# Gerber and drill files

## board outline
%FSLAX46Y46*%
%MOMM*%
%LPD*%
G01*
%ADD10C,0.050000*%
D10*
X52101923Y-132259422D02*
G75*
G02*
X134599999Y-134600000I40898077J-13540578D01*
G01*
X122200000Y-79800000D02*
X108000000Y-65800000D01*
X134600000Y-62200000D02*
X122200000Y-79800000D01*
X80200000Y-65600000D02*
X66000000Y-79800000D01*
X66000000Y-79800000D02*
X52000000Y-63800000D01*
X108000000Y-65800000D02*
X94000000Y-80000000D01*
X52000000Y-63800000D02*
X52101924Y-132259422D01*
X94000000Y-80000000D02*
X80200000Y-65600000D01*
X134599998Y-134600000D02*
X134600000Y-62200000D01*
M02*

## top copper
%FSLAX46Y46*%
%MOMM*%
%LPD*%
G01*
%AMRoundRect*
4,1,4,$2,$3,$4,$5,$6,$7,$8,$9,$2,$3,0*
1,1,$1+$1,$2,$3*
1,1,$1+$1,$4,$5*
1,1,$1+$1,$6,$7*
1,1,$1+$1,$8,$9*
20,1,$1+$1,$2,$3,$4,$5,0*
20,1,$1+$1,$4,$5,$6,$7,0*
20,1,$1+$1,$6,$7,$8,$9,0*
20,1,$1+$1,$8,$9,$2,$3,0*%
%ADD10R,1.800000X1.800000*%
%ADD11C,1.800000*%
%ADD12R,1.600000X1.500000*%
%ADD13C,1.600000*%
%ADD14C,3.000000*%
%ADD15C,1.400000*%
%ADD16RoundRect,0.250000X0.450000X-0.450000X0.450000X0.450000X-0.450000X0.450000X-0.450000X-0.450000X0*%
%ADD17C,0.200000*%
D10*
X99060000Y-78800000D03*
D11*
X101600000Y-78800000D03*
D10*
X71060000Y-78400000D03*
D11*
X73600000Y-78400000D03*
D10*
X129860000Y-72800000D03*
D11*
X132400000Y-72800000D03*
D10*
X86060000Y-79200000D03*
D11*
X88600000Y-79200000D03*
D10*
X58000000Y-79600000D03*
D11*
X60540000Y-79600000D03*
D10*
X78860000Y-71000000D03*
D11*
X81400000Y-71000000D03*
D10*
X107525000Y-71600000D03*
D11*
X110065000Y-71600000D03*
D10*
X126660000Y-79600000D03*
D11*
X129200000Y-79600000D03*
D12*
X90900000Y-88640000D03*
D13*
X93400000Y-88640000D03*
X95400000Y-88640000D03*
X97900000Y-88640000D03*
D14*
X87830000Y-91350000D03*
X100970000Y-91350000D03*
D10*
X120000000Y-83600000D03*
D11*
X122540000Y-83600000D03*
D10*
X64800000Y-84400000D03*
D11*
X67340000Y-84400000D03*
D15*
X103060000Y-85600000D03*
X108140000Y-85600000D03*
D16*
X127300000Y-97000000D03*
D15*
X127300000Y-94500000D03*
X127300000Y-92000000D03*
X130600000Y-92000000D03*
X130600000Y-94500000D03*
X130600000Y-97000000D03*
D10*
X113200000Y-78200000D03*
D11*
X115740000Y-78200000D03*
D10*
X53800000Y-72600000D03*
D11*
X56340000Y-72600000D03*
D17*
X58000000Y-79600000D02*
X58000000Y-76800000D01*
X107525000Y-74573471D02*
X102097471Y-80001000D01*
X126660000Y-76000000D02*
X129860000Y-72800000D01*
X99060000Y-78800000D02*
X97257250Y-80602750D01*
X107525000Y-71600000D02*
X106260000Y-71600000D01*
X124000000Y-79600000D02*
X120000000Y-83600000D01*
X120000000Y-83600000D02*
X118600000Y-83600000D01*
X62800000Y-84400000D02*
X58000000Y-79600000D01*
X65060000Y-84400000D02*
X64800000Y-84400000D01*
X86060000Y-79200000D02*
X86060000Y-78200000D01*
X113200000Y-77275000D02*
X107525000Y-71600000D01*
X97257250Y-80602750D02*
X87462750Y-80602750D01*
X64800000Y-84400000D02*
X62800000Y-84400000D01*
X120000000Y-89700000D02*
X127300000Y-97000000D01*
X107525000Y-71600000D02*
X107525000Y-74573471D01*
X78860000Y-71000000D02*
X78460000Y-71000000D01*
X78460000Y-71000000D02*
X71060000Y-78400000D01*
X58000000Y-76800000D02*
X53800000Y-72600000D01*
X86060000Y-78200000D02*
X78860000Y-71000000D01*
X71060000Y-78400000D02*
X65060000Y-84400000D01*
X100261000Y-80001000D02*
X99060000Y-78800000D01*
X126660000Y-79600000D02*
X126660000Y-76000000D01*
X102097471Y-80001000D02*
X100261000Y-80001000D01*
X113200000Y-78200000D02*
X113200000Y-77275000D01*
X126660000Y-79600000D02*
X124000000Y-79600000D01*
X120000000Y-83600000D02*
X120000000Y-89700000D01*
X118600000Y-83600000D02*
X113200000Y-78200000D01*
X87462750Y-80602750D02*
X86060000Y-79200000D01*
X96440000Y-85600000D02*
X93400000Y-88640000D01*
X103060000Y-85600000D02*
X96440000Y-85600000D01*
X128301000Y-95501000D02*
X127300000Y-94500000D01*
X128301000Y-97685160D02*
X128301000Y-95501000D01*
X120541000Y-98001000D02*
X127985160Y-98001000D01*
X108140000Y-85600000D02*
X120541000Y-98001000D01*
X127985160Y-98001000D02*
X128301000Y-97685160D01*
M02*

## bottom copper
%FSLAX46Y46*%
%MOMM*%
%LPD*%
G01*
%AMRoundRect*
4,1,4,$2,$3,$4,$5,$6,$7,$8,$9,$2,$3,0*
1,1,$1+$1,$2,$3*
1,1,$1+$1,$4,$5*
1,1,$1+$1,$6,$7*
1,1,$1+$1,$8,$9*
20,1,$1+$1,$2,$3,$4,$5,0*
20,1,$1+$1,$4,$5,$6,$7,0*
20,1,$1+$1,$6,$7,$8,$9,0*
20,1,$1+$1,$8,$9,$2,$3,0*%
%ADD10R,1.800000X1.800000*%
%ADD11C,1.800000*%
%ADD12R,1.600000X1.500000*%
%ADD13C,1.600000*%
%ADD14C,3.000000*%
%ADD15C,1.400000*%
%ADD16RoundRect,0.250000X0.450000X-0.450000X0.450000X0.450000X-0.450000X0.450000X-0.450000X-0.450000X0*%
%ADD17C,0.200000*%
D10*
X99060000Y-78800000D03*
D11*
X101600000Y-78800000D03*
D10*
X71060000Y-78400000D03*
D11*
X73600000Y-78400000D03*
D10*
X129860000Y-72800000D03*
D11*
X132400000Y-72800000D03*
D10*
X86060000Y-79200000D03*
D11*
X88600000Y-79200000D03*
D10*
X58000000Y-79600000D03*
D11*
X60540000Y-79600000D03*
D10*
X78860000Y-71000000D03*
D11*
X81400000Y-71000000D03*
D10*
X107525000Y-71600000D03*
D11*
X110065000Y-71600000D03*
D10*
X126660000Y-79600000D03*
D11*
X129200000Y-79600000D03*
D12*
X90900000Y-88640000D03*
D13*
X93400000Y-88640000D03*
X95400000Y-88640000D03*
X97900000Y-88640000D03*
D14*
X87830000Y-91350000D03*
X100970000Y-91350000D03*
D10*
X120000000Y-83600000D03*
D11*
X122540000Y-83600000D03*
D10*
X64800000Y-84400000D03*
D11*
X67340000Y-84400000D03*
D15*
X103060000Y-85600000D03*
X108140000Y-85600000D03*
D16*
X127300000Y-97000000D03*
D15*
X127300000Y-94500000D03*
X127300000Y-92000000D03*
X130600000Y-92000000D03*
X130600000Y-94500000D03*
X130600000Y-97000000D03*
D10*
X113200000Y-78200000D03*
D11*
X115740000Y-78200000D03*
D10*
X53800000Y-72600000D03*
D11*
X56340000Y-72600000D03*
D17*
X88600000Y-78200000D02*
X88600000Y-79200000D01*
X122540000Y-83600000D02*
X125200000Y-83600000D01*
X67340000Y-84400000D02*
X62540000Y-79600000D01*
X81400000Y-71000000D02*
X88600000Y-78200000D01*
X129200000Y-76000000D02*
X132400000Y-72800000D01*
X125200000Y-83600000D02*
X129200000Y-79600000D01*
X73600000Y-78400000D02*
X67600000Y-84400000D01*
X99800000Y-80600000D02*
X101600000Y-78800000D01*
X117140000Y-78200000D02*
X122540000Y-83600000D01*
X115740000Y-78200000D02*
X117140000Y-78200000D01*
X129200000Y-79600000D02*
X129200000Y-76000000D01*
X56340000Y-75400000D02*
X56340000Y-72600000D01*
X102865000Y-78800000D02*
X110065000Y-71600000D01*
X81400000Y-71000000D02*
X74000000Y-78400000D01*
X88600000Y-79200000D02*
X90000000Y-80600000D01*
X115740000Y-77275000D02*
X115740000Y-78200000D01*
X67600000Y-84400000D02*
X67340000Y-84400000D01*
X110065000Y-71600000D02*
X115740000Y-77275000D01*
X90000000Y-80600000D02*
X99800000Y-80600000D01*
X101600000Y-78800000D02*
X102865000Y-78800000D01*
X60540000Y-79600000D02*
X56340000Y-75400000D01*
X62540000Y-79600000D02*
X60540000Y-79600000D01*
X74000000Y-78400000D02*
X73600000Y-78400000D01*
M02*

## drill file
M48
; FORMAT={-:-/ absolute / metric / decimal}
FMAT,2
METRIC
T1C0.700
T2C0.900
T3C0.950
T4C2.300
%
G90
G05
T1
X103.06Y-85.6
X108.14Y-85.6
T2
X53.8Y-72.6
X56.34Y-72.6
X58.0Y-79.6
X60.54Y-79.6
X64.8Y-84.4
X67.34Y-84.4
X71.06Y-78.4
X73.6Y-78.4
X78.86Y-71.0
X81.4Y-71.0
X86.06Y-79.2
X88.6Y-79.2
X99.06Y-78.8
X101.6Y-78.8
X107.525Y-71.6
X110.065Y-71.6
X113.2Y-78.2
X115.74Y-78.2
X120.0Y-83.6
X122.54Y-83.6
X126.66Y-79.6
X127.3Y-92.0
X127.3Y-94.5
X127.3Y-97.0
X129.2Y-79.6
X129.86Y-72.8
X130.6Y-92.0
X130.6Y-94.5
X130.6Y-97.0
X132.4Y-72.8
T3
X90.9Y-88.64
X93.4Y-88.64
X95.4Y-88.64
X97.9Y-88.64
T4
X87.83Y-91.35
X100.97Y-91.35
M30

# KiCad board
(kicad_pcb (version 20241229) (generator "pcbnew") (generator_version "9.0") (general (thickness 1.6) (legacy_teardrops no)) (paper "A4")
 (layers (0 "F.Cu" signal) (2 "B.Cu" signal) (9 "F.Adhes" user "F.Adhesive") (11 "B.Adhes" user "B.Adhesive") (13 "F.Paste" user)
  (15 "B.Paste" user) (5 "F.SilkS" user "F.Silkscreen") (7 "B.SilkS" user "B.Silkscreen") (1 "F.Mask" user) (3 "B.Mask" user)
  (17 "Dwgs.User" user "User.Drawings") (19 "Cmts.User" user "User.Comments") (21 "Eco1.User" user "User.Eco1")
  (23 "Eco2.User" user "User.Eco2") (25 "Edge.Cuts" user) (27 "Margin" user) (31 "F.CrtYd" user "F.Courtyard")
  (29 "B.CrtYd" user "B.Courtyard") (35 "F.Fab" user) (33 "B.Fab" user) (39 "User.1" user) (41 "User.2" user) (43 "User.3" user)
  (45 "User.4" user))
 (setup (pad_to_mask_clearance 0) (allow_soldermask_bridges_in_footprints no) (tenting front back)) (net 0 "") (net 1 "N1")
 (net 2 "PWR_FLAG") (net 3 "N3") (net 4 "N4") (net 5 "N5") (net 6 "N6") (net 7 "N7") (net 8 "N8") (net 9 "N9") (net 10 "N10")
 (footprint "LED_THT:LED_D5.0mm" (layer "F.Cu") (at 99.06 78.8)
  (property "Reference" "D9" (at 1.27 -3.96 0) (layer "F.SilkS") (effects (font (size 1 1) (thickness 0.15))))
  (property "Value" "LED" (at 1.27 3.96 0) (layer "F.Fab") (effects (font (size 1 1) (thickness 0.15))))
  (pad "1" thru_hole rect (at 0 0) (size 1.8 1.8) (drill 0.9) (layers "*.Cu" "*.Mask") (remove_unused_layers no) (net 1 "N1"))
  (pad "2" thru_hole circle (at 2.54 0) (size 1.8 1.8) (drill 0.9) (layers "*.Cu" "*.Mask") (remove_unused_layers no) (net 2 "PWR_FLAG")))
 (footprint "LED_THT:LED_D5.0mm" (layer "F.Cu") (at 71.06 78.4)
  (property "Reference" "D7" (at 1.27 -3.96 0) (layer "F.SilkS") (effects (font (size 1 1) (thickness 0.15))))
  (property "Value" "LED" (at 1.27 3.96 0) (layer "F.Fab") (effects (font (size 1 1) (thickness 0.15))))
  (pad "1" thru_hole rect (at 0 0) (size 1.8 1.8) (drill 0.9) (layers "*.Cu" "*.Mask") (remove_unused_layers no) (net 1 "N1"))
  (pad "2" thru_hole circle (at 2.54 0) (size 1.8 1.8) (drill 0.9) (layers "*.Cu" "*.Mask") (remove_unused_layers no) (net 2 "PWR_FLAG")))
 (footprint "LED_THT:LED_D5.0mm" (layer "F.Cu") (at 129.86 72.8)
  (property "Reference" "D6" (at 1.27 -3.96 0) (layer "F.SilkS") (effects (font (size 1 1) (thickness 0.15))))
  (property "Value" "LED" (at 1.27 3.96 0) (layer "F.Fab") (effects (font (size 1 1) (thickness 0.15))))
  (pad "1" thru_hole rect (at 0 0) (size 1.8 1.8) (drill 0.9) (layers "*.Cu" "*.Mask") (remove_unused_layers no) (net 1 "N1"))
  (pad "2" thru_hole circle (at 2.54 0) (size 1.8 1.8) (drill 0.9) (layers "*.Cu" "*.Mask") (remove_unused_layers no) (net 2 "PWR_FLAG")))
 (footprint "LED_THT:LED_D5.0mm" (layer "F.Cu") (at 86.06 79.2)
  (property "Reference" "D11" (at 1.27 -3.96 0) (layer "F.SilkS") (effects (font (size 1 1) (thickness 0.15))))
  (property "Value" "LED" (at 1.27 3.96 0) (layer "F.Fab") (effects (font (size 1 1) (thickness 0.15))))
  (pad "1" thru_hole rect (at 0 0) (size 1.8 1.8) (drill 0.9) (layers "*.Cu" "*.Mask") (remove_unused_layers no) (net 1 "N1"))
  (pad "2" thru_hole circle (at 2.54 0) (size 1.8 1.8) (drill 0.9) (layers "*.Cu" "*.Mask") (remove_unused_layers no) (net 2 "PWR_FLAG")))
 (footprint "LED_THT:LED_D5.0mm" (layer "F.Cu") (at 58 79.6)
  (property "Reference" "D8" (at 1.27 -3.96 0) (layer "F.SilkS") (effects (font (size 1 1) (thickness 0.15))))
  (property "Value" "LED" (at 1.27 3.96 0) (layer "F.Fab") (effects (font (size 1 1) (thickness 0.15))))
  (pad "1" thru_hole rect (at 0 0) (size 1.8 1.8) (drill 0.9) (layers "*.Cu" "*.Mask") (remove_unused_layers no) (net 1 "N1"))
  (pad "2" thru_hole circle (at 2.54 0) (size 1.8 1.8) (drill 0.9) (layers "*.Cu" "*.Mask") (remove_unused_layers no) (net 2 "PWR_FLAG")))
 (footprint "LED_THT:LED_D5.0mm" (layer "F.Cu") (at 78.86 71)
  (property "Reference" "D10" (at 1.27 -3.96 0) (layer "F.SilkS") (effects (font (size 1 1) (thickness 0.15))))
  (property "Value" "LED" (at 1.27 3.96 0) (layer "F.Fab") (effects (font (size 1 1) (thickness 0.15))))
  (pad "1" thru_hole rect (at 0 0) (size 1.8 1.8) (drill 0.9) (layers "*.Cu" "*.Mask") (remove_unused_layers no) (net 1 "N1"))
  (pad "2" thru_hole circle (at 2.54 0) (size 1.8 1.8) (drill 0.9) (layers "*.Cu" "*.Mask") (remove_unused_layers no) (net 2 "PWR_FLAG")))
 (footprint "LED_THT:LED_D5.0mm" (layer "F.Cu") (at 107.525 71.6)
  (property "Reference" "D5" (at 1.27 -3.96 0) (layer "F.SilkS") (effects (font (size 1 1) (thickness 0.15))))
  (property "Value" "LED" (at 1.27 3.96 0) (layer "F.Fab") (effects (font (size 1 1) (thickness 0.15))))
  (pad "1" thru_hole rect (at 0 0) (size 1.8 1.8) (drill 0.9) (layers "*.Cu" "*.Mask") (remove_unused_layers no) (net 1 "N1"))
  (pad "2" thru_hole circle (at 2.54 0) (size 1.8 1.8) (drill 0.9) (layers "*.Cu" "*.Mask") (remove_unused_layers no) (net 2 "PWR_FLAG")))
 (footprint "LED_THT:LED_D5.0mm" (layer "F.Cu") (at 126.66 79.6)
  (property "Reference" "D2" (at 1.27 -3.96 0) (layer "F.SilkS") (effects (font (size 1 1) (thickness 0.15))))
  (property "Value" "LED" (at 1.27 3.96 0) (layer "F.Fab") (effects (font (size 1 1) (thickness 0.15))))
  (pad "1" thru_hole rect (at 0 0) (size 1.8 1.8) (drill 0.9) (layers "*.Cu" "*.Mask") (remove_unused_layers no) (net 1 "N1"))
  (pad "2" thru_hole circle (at 2.54 0) (size 1.8 1.8) (drill 0.9) (layers "*.Cu" "*.Mask") (remove_unused_layers no) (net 2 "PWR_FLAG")))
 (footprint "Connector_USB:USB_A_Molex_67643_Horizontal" (layer "F.Cu") (at 90.9 88.64)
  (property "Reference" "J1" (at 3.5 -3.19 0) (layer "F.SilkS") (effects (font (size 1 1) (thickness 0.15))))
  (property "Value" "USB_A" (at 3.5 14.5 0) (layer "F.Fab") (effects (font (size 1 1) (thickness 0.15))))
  (pad "1" thru_hole rect (at 0 0) (size 1.6 1.5) (drill 0.95) (layers "*.Cu" "*.Mask") (remove_unused_layers no) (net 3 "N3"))
  (pad "2" thru_hole circle (at 2.5 0) (size 1.6 1.6) (drill 0.95) (layers "*.Cu" "*.Mask") (remove_unused_layers no) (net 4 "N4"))
  (pad "3" thru_hole circle (at 4.5 0) (size 1.6 1.6) (drill 0.95) (layers "*.Cu" "*.Mask") (remove_unused_layers no) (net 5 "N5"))
  (pad "4" thru_hole circle (at 7 0) (size 1.6 1.6) (drill 0.95) (layers "*.Cu" "*.Mask") (remove_unused_layers no) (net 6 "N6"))
  (pad "5" thru_hole circle (at -3.07 2.71) (size 3 3) (drill 2.3) (layers "*.Cu" "*.Mask") (remove_unused_layers no) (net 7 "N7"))
  (pad "5" thru_hole circle (at 10.07 2.71) (size 3 3) (drill 2.3) (layers "*.Cu" "*.Mask") (remove_unused_layers no) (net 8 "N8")))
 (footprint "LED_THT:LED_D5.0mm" (layer "F.Cu") (at 120 83.6)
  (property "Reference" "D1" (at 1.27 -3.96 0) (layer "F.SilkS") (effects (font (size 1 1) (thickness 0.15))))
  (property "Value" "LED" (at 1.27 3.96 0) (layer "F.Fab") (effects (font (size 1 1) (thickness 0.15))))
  (pad "1" thru_hole rect (at 0 0) (size 1.8 1.8) (drill 0.9) (layers "*.Cu" "*.Mask") (remove_unused_layers no) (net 1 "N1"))
  (pad "2" thru_hole circle (at 2.54 0) (size 1.8 1.8) (drill 0.9) (layers "*.Cu" "*.Mask") (remove_unused_layers no) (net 2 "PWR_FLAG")))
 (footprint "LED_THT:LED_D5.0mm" (layer "F.Cu") (at 64.8 84.4)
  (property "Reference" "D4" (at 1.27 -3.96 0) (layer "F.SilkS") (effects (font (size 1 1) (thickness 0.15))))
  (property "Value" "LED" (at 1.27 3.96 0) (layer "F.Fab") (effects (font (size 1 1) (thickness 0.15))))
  (pad "1" thru_hole rect (at 0 0) (size 1.8 1.8) (drill 0.9) (layers "*.Cu" "*.Mask") (remove_unused_layers no) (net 1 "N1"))
  (pad "2" thru_hole circle (at 2.54 0) (size 1.8 1.8) (drill 0.9) (layers "*.Cu" "*.Mask") (remove_unused_layers no) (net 2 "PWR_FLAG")))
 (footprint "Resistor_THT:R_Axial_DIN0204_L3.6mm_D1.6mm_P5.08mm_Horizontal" (layer "F.Cu") (at 103.06 85.6)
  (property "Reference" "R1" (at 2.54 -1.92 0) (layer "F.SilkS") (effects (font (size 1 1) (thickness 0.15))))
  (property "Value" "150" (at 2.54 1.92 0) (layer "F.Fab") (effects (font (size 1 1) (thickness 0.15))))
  (pad "1" thru_hole circle (at 0 0) (size 1.4 1.4) (drill 0.7) (layers "*.Cu" "*.Mask") (remove_unused_layers no) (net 4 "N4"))
  (pad "2" thru_hole circle (at 5.08 0) (size 1.4 1.4) (drill 0.7) (layers "*.Cu" "*.Mask") (remove_unused_layers no) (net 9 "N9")))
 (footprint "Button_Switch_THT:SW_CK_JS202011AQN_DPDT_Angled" (layer "F.Cu") (at 127.3 97 90)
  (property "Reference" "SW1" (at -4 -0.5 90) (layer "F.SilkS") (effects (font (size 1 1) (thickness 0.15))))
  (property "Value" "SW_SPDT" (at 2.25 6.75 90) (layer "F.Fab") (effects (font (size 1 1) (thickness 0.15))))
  (pad "1" thru_hole roundrect (at 0 0 90) (size 1.4 1.4) (drill 0.9) (layers "*.Cu" "*.Mask") (remove_unused_layers no)
   (roundrect_rratio 0.1785714286) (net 1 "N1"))
  (pad "2" thru_hole circle (at 2.5 0 90) (size 1.4 1.4) (drill 0.9) (layers "*.Cu" "*.Mask") (remove_unused_layers no) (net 9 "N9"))
  (pad "3" thru_hole circle (at 5 0 90) (size 1.4 1.4) (drill 0.9) (layers "*.Cu" "*.Mask") (remove_unused_layers no) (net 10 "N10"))
  (pad "4" thru_hole circle (at 5 3.3 90) (size 1.4 1.4) (drill 0.9) (layers "*.Cu" "*.Mask") (remove_unused_layers no))
  (pad "5" thru_hole circle (at 2.5 3.3 90) (size 1.4 1.4) (drill 0.9) (layers "*.Cu" "*.Mask") (remove_unused_layers no))
  (pad "6" thru_hole circle (at 0 3.3 90) (size 1.4 1.4) (drill 0.9) (layers "*.Cu" "*.Mask") (remove_unused_layers no)))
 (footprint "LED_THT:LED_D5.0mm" (layer "F.Cu") (at 113.2 78.2)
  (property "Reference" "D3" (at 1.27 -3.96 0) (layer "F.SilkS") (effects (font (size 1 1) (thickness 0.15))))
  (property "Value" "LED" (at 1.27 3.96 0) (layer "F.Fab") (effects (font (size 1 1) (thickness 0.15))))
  (pad "1" thru_hole rect (at 0 0) (size 1.8 1.8) (drill 0.9) (layers "*.Cu" "*.Mask") (remove_unused_layers no) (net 1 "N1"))
  (pad "2" thru_hole circle (at 2.54 0) (size 1.8 1.8) (drill 0.9) (layers "*.Cu" "*.Mask") (remove_unused_layers no) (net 2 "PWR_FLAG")))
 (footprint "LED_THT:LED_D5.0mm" (layer "F.Cu") (at 53.8 72.6)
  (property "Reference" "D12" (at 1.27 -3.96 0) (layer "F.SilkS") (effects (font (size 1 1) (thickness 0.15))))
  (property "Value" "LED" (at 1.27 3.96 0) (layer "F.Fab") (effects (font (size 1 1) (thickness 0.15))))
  (pad "1" thru_hole rect (at 0 0) (size 1.8 1.8) (drill 0.9) (layers "*.Cu" "*.Mask") (remove_unused_layers no) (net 1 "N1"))
  (pad "2" thru_hole circle (at 2.54 0) (size 1.8 1.8) (drill 0.9) (layers "*.Cu" "*.Mask") (remove_unused_layers no) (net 2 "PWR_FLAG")))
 (gr_arc (start 52.101923 132.259422) (mid 94.221782 102.73601) (end 134.6 134.6) (stroke (width 0.05) (type default)) (layer "Edge.Cuts"))
 (gr_line (start 122.2 79.8) (end 108 65.8) (stroke (width 0.05) (type default)) (layer "Edge.Cuts"))
 (gr_line (start 134.6 62.2) (end 122.2 79.8) (stroke (width 0.05) (type default)) (layer "Edge.Cuts"))
 (gr_line (start 80.2 65.6) (end 66 79.8) (stroke (width 0.05) (type default)) (layer "Edge.Cuts"))
 (gr_line (start 66 79.8) (end 52 63.8) (stroke (width 0.05) (type default)) (layer "Edge.Cuts"))
 (gr_line (start 108 65.8) (end 94 80) (stroke (width 0.05) (type default)) (layer "Edge.Cuts"))
 (gr_line (start 52 63.8) (end 52.101924 132.259422) (stroke (width 0.05) (type default)) (layer "Edge.Cuts"))
 (gr_line (start 94 80) (end 80.2 65.6) (stroke (width 0.05) (type default)) (layer "Edge.Cuts"))
 (gr_line (start 134.599998 134.6) (end 134.6 62.2) (stroke (width 0.05) (type default)) (layer "Edge.Cuts"))
 (segment (start 88.6 78.2) (end 88.6 79.2) (width 0.2) (layer "B.Cu") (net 2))
 (segment (start 122.54 83.6) (end 125.2 83.6) (width 0.2) (layer "B.Cu") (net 2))
 (segment (start 67.34 84.4) (end 62.54 79.6) (width 0.2) (layer "B.Cu") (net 2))
 (segment (start 81.4 71) (end 88.6 78.2) (width 0.2) (layer "B.Cu") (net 2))
 (segment (start 129.2 76) (end 132.4 72.8) (width 0.2) (layer "B.Cu") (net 2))
 (segment (start 125.2 83.6) (end 129.2 79.6) (width 0.2) (layer "B.Cu") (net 2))
 (segment (start 73.6 78.4) (end 67.6 84.4) (width 0.2) (layer "B.Cu") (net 2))
 (segment (start 99.8 80.6) (end 101.6 78.8) (width 0.2) (layer "B.Cu") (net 2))
 (segment (start 117.14 78.2) (end 122.54 83.6) (width 0.2) (layer "B.Cu") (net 2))
 (segment (start 115.74 78.2) (end 117.14 78.2) (width 0.2) (layer "B.Cu") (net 2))
 (segment (start 129.2 79.6) (end 129.2 76) (width 0.2) (layer "B.Cu") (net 2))
 (segment (start 56.34 75.4) (end 56.34 72.6) (width 0.2) (layer "B.Cu") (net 2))
 (segment (start 102.865 78.8) (end 110.065 71.6) (width 0.2) (layer "B.Cu") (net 2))
 (segment (start 81.4 71) (end 74 78.4) (width 0.2) (layer "B.Cu") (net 2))
 (segment (start 88.6 79.2) (end 90 80.6) (width 0.2) (layer "B.Cu") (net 2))
 (segment (start 115.74 77.275) (end 115.74 78.2) (width 0.2) (layer "B.Cu") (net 2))
 (segment (start 67.6 84.4) (end 67.34 84.4) (width 0.2) (layer "B.Cu") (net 2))
 (segment (start 110.065 71.6) (end 115.74 77.275) (width 0.2) (layer "B.Cu") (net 2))
 (segment (start 90 80.6) (end 99.8 80.6) (width 0.2) (layer "B.Cu") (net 2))
 (segment (start 101.6 78.8) (end 102.865 78.8) (width 0.2) (layer "B.Cu") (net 2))
 (segment (start 60.54 79.6) (end 56.34 75.4) (width 0.2) (layer "B.Cu") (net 2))
 (segment (start 62.54 79.6) (end 60.54 79.6) (width 0.2) (layer "B.Cu") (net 2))
 (segment (start 74 78.4) (end 73.6 78.4) (width 0.2) (layer "B.Cu") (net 2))
 (segment (start 58 79.6) (end 58 76.8) (width 0.2) (layer "F.Cu") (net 1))
 (segment (start 107.525 74.573471) (end 102.097471 80.001) (width 0.2) (layer "F.Cu") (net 1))
 (segment (start 126.66 76) (end 129.86 72.8) (width 0.2) (layer "F.Cu") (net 1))
 (segment (start 99.06 78.8) (end 97.25725 80.60275) (width 0.2) (layer "F.Cu") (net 1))
 (segment (start 107.525 71.6) (end 106.26 71.6) (width 0.2) (layer "F.Cu") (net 1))
 (segment (start 124 79.6) (end 120 83.6) (width 0.2) (layer "F.Cu") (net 1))
 (segment (start 120 83.6) (end 118.6 83.6) (width 0.2) (layer "F.Cu") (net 1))
 (segment (start 62.8 84.4) (end 58 79.6) (width 0.2) (layer "F.Cu") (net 1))
 (segment (start 65.06 84.4) (end 64.8 84.4) (width 0.2) (layer "F.Cu") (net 1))
 (segment (start 86.06 79.2) (end 86.06 78.2) (width 0.2) (layer "F.Cu") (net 1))
 (segment (start 113.2 77.275) (end 107.525 71.6) (width 0.2) (layer "F.Cu") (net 1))
 (segment (start 97.25725 80.60275) (end 87.46275 80.60275) (width 0.2) (layer "F.Cu") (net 1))
 (segment (start 64.8 84.4) (end 62.8 84.4) (width 0.2) (layer "F.Cu") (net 1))
 (segment (start 120 89.7) (end 127.3 97) (width 0.2) (layer "F.Cu") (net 1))
 (segment (start 107.525 71.6) (end 107.525 74.573471) (width 0.2) (layer "F.Cu") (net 1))
 (segment (start 78.86 71) (end 78.46 71) (width 0.2) (layer "F.Cu") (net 1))
 (segment (start 78.46 71) (end 71.06 78.4) (width 0.2) (layer "F.Cu") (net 1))
 (segment (start 58 76.8) (end 53.8 72.6) (width 0.2) (layer "F.Cu") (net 1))
 (segment (start 86.06 78.2) (end 78.86 71) (width 0.2) (layer "F.Cu") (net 1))
 (segment (start 71.06 78.4) (end 65.06 84.4) (width 0.2) (layer "F.Cu") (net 1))
 (segment (start 100.261 80.001) (end 99.06 78.8) (width 0.2) (layer "F.Cu") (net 1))
 (segment (start 126.66 79.6) (end 126.66 76) (width 0.2) (layer "F.Cu") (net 1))
 (segment (start 102.097471 80.001) (end 100.261 80.001) (width 0.2) (layer "F.Cu") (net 1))
 (segment (start 113.2 78.2) (end 113.2 77.275) (width 0.2) (layer "F.Cu") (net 1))
 (segment (start 126.66 79.6) (end 124 79.6) (width 0.2) (layer "F.Cu") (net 1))
 (segment (start 120 83.6) (end 120 89.7) (width 0.2) (layer "F.Cu") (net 1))
 (segment (start 118.6 83.6) (end 113.2 78.2) (width 0.2) (layer "F.Cu") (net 1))
 (segment (start 87.46275 80.60275) (end 86.06 79.2) (width 0.2) (layer "F.Cu") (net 1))
 (segment (start 96.44 85.6) (end 93.4 88.64) (width 0.2) (layer "F.Cu") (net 4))
 (segment (start 103.06 85.6) (end 96.44 85.6) (width 0.2) (layer "F.Cu") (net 4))
 (segment (start 128.301 95.501) (end 127.3 94.5) (width 0.2) (layer "F.Cu") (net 9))
 (segment (start 128.301 97.68516) (end 128.301 95.501) (width 0.2) (layer "F.Cu") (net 9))
 (segment (start 120.541 98.001) (end 127.98516 98.001) (width 0.2) (layer "F.Cu") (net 9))
 (segment (start 108.14 85.6) (end 120.541 98.001) (width 0.2) (layer "F.Cu") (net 9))
 (segment (start 127.98516 98.001) (end 128.301 97.68516) (width 0.2) (layer "F.Cu") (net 9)))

